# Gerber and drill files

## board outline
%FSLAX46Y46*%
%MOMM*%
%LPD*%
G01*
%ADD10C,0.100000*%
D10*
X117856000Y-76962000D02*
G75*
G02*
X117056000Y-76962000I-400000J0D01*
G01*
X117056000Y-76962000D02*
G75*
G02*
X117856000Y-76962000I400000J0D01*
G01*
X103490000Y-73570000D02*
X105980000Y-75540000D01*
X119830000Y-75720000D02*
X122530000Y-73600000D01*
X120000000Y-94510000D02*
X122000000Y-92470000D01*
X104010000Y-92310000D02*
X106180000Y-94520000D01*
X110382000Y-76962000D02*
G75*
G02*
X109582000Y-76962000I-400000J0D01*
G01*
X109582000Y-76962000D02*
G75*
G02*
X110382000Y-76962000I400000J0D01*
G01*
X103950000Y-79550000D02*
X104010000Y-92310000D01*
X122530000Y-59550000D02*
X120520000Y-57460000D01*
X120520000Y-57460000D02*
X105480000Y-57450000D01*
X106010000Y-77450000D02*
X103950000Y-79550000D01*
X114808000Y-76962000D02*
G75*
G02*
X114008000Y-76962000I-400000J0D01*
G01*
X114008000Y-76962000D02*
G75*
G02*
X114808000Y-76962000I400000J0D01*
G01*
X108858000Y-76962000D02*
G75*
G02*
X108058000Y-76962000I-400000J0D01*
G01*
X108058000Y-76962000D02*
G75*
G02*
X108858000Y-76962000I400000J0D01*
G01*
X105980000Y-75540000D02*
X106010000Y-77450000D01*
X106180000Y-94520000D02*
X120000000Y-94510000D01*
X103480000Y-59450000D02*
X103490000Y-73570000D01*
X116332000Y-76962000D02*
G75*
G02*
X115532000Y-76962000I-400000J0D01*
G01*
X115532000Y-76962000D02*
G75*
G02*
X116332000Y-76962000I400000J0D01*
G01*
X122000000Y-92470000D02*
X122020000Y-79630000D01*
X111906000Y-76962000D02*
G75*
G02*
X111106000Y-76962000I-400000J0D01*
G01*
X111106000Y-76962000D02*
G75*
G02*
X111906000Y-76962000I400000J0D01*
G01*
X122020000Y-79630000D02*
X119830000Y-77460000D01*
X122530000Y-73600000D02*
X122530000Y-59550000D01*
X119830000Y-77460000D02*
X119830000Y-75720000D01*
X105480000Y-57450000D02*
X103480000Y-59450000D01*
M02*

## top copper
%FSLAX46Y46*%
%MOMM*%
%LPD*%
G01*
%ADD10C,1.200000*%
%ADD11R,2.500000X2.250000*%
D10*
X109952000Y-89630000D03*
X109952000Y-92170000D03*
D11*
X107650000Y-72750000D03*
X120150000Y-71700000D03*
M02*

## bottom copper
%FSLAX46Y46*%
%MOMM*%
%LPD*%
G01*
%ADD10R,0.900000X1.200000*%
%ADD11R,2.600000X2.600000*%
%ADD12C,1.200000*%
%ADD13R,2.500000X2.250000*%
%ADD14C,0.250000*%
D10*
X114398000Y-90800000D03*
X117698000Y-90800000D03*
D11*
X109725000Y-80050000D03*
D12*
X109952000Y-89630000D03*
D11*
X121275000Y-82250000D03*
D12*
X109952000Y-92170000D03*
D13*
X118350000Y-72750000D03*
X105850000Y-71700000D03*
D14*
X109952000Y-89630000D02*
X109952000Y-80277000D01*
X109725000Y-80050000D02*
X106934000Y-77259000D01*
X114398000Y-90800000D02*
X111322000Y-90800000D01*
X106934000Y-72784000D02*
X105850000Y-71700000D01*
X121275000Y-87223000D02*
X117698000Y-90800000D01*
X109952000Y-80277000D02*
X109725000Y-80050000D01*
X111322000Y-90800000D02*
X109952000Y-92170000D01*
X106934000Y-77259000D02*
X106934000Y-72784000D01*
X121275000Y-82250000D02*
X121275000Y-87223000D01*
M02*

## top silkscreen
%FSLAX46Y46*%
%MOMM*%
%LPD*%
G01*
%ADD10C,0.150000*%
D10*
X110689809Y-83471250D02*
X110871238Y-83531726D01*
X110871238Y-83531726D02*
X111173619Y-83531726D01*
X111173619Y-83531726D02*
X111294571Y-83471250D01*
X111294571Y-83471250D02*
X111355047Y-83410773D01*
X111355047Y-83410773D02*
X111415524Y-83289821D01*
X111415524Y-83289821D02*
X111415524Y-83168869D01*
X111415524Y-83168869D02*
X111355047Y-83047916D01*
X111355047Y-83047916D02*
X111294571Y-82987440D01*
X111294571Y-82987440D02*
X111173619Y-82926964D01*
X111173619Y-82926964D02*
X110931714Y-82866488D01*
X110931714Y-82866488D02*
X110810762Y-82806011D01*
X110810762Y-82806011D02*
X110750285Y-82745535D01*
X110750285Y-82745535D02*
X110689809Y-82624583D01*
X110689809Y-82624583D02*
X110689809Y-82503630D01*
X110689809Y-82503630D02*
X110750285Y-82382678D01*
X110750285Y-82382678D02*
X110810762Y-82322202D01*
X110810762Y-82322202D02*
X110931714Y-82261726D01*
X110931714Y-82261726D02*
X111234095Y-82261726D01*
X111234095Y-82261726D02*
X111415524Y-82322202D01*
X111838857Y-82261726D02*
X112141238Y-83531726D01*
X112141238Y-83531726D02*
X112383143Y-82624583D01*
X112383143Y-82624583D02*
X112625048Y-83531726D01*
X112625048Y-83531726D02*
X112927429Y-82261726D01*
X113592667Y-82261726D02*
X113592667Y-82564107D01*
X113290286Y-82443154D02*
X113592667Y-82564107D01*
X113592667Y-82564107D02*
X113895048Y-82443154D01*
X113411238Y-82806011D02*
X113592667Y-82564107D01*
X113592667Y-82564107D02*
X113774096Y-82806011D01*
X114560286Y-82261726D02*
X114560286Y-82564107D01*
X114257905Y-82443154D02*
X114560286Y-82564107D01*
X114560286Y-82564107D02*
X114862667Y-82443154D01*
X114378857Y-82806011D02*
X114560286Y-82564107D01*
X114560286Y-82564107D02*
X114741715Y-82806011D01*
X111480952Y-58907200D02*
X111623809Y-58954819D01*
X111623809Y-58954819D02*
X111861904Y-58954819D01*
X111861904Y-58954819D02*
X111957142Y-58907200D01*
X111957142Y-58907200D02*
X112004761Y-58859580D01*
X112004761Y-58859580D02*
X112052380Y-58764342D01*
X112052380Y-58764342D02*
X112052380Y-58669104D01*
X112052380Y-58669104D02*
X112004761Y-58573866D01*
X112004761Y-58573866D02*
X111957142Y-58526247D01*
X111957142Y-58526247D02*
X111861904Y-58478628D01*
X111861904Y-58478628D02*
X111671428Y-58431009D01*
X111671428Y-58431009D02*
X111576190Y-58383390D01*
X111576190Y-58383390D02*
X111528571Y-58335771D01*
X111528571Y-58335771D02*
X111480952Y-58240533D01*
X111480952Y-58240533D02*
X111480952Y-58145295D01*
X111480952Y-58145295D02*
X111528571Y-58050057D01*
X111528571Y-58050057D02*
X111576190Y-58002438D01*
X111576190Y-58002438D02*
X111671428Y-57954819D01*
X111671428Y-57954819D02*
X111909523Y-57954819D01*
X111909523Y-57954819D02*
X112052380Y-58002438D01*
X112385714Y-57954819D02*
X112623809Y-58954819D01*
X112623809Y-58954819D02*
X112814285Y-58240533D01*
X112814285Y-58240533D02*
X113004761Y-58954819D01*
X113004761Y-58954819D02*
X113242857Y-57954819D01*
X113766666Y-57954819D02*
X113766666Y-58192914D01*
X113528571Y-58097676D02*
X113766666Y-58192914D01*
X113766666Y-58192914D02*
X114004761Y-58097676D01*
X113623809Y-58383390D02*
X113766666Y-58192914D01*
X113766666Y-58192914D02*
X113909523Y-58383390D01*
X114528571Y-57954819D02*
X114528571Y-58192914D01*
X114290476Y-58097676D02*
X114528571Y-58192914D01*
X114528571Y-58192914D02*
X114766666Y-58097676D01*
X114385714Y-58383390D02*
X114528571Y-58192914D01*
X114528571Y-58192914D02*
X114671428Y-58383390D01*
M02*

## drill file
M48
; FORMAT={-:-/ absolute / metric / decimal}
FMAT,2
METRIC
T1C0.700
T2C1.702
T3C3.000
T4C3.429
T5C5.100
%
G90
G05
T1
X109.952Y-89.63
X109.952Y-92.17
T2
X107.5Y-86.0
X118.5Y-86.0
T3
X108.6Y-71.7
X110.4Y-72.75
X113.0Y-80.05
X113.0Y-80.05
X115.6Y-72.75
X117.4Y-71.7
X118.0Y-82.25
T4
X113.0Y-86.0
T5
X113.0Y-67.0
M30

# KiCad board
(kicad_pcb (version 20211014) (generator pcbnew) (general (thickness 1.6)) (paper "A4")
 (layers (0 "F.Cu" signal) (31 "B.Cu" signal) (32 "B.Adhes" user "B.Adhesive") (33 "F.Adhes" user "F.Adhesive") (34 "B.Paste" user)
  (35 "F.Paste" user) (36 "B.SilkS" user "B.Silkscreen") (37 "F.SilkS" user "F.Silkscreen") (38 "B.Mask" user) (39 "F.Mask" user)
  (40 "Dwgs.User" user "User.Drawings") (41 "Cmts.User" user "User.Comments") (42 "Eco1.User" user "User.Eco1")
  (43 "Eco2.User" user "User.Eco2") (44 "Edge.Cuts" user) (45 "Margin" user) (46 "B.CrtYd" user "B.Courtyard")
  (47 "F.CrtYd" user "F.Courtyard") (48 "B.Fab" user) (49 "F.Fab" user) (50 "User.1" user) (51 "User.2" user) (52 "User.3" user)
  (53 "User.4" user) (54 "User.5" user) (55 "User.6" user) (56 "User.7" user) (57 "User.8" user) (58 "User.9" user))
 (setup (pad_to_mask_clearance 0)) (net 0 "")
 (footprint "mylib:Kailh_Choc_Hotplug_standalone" (layer "F.Cu") (at 113 86)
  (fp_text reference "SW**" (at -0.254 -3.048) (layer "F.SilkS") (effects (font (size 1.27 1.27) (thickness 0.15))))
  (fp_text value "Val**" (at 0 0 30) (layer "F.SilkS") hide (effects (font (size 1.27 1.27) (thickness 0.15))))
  (pad "" np_thru_hole circle (at 0 -5.95 30) (size 3 3) (drill 3) (layers *.Cu *.Mask))
  (pad "" np_thru_hole circle (at 5.5 0 30) (size 1.7018 1.7018) (drill 1.7018) (layers *.Cu *.Mask))
  (pad "" np_thru_hole circle (at 0 -5.95 30) (size 3 3) (drill 3) (layers *.Cu *.Mask))
  (pad "" np_thru_hole circle (at 0 0 30) (size 3.429 3.429) (drill 3.429) (layers *.Cu *.Mask))
  (pad "" np_thru_hole circle (at -5.5 0 30) (size 1.7018 1.7018) (drill 1.7018) (layers *.Cu *.Mask))
  (pad "" smd rect (at 1.398 4.8) (size 0.9 1.2) (layers "B.Cu" "B.Mask"))
  (pad "" np_thru_hole circle (at 5 -3.75 30) (size 3 3) (drill 3) (layers *.Cu *.Mask))
  (pad "" smd rect (at 4.698 4.8) (size 0.9 1.2) (layers "B.Cu" "B.Mask"))
  (pad "1" smd rect (at -3.275 -5.95) (size 2.6 2.6) (layers "B.Cu" "B.Mask"))
  (pad "1" thru_hole circle (at -3.048 3.63) (size 1.2 1.2) (drill 0.7) (layers *.Cu *.Mask))
  (pad "2" smd rect (at 8.275 -3.75) (size 2.6 2.6) (layers "B.Cu" "B.Mask"))
  (pad "2" thru_hole circle (at -3.048 6.17) (size 1.2 1.2) (drill 0.7) (layers *.Cu *.Mask)))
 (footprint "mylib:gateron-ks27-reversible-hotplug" (layer "F.Cu") (at 113 67)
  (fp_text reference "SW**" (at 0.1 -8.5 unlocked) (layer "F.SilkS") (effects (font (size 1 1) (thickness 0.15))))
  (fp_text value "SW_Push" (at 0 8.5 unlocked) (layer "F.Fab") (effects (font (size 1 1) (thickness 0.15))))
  (pad "" np_thru_hole circle (at -2.6 5.75) (size 3 3) (drill 3) (layers *.Mask))
  (pad "" np_thru_hole circle (at 2.6 5.75) (size 3 3) (drill 3) (layers *.Mask))
  (pad "" np_thru_hole circle (at 4.4 4.7) (size 3 3) (drill 3) (layers *.Mask))
  (pad "" np_thru_hole circle (at -4.4 4.7) (size 3 3) (drill 3) (layers *.Mask))
  (pad "" np_thru_hole circle (at 0 0) (size 5.1 5.1) (drill 5.1) (layers F&B.Cu *.Mask))
  (pad "1" smd rect (at -5.35 5.75) (size 2.5 2.25) (layers "F.Cu" "F.Mask"))
  (pad "1" smd rect (at 5.35 5.75) (size 2.5 2.25) (layers "B.Cu" "B.Mask"))
  (pad "2" smd rect (at 7.15 4.7) (size 2.5 2.25) (layers "F.Cu" "F.Mask"))
  (pad "2" smd rect (at -7.15 4.7) (size 2.5 2.25) (layers "B.Cu" "B.Mask")))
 (gr_circle (center 117.456 76.962) (end 117.856 76.962) (layer "Edge.Cuts") (width 0.1) (fill none))
 (gr_line (start 103.49 73.57) (end 105.98 75.54) (layer "Edge.Cuts") (width 0.1))
 (gr_line (start 119.83 75.72) (end 122.53 73.6) (layer "Edge.Cuts") (width 0.1))
 (gr_line (start 120 94.51) (end 122 92.47) (layer "Edge.Cuts") (width 0.1))
 (gr_line (start 104.01 92.31) (end 106.18 94.52) (layer "Edge.Cuts") (width 0.1))
 (gr_circle (center 109.982 76.962) (end 110.382 76.962) (layer "Edge.Cuts") (width 0.1) (fill none))
 (gr_line (start 103.95 79.55) (end 104.01 92.31) (layer "Edge.Cuts") (width 0.1))
 (gr_line (start 122.53 59.55) (end 120.52 57.46) (layer "Edge.Cuts") (width 0.1))
 (gr_line (start 120.52 57.46) (end 105.48 57.45) (layer "Edge.Cuts") (width 0.1))
 (gr_line (start 106.01 77.45) (end 103.95 79.55) (layer "Edge.Cuts") (width 0.1))
 (gr_circle (center 114.408 76.962) (end 114.808 76.962) (layer "Edge.Cuts") (width 0.1) (fill none))
 (gr_circle (center 108.458 76.962) (end 108.858 76.962) (layer "Edge.Cuts") (width 0.1) (fill none))
 (gr_line (start 105.98 75.54) (end 106.01 77.45) (layer "Edge.Cuts") (width 0.1))
 (gr_line (start 106.18 94.52) (end 120 94.51) (layer "Edge.Cuts") (width 0.1))
 (gr_line (start 103.48 59.45) (end 103.49 73.57) (layer "Edge.Cuts") (width 0.1))
 (gr_circle (center 115.932 76.962) (end 116.332 76.962) (layer "Edge.Cuts") (width 0.1) (fill none))
 (gr_line (start 122 92.47) (end 122.02 79.63) (layer "Edge.Cuts") (width 0.1))
 (gr_circle (center 111.506 76.962) (end 111.906 76.962) (layer "Edge.Cuts") (width 0.1) (fill none))
 (gr_line (start 122.02 79.63) (end 119.83 77.46) (layer "Edge.Cuts") (width 0.1))
 (gr_line (start 122.53 73.6) (end 122.53 59.55) (layer "Edge.Cuts") (width 0.1))
 (gr_line (start 119.83 77.46) (end 119.83 75.72) (layer "Edge.Cuts") (width 0.1))
 (gr_line (start 105.48 57.45) (end 103.48 59.45) (layer "Edge.Cuts") (width 0.1))
 (segment (start 109.952 89.63) (end 109.952 80.277) (width 0.25) (layer "B.Cu") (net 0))
 (segment (start 109.725 80.05) (end 106.934 77.259) (width 0.25) (layer "B.Cu") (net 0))
 (segment (start 114.398 90.8) (end 111.322 90.8) (width 0.25) (layer "B.Cu") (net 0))
 (segment (start 106.934 72.784) (end 105.85 71.7) (width 0.25) (layer "B.Cu") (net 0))
 (segment (start 121.275 87.223) (end 117.698 90.8) (width 0.25) (layer "B.Cu") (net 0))
 (segment (start 109.952 80.277) (end 109.725 80.05) (width 0.25) (layer "B.Cu") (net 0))
 (segment (start 111.322 90.8) (end 109.952 92.17) (width 0.25) (layer "B.Cu") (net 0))
 (segment (start 106.934 77.259) (end 106.934 72.784) (width 0.25) (layer "B.Cu") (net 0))
 (segment (start 121.275 82.25) (end 121.275 87.223) (width 0.25) (layer "B.Cu") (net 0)))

